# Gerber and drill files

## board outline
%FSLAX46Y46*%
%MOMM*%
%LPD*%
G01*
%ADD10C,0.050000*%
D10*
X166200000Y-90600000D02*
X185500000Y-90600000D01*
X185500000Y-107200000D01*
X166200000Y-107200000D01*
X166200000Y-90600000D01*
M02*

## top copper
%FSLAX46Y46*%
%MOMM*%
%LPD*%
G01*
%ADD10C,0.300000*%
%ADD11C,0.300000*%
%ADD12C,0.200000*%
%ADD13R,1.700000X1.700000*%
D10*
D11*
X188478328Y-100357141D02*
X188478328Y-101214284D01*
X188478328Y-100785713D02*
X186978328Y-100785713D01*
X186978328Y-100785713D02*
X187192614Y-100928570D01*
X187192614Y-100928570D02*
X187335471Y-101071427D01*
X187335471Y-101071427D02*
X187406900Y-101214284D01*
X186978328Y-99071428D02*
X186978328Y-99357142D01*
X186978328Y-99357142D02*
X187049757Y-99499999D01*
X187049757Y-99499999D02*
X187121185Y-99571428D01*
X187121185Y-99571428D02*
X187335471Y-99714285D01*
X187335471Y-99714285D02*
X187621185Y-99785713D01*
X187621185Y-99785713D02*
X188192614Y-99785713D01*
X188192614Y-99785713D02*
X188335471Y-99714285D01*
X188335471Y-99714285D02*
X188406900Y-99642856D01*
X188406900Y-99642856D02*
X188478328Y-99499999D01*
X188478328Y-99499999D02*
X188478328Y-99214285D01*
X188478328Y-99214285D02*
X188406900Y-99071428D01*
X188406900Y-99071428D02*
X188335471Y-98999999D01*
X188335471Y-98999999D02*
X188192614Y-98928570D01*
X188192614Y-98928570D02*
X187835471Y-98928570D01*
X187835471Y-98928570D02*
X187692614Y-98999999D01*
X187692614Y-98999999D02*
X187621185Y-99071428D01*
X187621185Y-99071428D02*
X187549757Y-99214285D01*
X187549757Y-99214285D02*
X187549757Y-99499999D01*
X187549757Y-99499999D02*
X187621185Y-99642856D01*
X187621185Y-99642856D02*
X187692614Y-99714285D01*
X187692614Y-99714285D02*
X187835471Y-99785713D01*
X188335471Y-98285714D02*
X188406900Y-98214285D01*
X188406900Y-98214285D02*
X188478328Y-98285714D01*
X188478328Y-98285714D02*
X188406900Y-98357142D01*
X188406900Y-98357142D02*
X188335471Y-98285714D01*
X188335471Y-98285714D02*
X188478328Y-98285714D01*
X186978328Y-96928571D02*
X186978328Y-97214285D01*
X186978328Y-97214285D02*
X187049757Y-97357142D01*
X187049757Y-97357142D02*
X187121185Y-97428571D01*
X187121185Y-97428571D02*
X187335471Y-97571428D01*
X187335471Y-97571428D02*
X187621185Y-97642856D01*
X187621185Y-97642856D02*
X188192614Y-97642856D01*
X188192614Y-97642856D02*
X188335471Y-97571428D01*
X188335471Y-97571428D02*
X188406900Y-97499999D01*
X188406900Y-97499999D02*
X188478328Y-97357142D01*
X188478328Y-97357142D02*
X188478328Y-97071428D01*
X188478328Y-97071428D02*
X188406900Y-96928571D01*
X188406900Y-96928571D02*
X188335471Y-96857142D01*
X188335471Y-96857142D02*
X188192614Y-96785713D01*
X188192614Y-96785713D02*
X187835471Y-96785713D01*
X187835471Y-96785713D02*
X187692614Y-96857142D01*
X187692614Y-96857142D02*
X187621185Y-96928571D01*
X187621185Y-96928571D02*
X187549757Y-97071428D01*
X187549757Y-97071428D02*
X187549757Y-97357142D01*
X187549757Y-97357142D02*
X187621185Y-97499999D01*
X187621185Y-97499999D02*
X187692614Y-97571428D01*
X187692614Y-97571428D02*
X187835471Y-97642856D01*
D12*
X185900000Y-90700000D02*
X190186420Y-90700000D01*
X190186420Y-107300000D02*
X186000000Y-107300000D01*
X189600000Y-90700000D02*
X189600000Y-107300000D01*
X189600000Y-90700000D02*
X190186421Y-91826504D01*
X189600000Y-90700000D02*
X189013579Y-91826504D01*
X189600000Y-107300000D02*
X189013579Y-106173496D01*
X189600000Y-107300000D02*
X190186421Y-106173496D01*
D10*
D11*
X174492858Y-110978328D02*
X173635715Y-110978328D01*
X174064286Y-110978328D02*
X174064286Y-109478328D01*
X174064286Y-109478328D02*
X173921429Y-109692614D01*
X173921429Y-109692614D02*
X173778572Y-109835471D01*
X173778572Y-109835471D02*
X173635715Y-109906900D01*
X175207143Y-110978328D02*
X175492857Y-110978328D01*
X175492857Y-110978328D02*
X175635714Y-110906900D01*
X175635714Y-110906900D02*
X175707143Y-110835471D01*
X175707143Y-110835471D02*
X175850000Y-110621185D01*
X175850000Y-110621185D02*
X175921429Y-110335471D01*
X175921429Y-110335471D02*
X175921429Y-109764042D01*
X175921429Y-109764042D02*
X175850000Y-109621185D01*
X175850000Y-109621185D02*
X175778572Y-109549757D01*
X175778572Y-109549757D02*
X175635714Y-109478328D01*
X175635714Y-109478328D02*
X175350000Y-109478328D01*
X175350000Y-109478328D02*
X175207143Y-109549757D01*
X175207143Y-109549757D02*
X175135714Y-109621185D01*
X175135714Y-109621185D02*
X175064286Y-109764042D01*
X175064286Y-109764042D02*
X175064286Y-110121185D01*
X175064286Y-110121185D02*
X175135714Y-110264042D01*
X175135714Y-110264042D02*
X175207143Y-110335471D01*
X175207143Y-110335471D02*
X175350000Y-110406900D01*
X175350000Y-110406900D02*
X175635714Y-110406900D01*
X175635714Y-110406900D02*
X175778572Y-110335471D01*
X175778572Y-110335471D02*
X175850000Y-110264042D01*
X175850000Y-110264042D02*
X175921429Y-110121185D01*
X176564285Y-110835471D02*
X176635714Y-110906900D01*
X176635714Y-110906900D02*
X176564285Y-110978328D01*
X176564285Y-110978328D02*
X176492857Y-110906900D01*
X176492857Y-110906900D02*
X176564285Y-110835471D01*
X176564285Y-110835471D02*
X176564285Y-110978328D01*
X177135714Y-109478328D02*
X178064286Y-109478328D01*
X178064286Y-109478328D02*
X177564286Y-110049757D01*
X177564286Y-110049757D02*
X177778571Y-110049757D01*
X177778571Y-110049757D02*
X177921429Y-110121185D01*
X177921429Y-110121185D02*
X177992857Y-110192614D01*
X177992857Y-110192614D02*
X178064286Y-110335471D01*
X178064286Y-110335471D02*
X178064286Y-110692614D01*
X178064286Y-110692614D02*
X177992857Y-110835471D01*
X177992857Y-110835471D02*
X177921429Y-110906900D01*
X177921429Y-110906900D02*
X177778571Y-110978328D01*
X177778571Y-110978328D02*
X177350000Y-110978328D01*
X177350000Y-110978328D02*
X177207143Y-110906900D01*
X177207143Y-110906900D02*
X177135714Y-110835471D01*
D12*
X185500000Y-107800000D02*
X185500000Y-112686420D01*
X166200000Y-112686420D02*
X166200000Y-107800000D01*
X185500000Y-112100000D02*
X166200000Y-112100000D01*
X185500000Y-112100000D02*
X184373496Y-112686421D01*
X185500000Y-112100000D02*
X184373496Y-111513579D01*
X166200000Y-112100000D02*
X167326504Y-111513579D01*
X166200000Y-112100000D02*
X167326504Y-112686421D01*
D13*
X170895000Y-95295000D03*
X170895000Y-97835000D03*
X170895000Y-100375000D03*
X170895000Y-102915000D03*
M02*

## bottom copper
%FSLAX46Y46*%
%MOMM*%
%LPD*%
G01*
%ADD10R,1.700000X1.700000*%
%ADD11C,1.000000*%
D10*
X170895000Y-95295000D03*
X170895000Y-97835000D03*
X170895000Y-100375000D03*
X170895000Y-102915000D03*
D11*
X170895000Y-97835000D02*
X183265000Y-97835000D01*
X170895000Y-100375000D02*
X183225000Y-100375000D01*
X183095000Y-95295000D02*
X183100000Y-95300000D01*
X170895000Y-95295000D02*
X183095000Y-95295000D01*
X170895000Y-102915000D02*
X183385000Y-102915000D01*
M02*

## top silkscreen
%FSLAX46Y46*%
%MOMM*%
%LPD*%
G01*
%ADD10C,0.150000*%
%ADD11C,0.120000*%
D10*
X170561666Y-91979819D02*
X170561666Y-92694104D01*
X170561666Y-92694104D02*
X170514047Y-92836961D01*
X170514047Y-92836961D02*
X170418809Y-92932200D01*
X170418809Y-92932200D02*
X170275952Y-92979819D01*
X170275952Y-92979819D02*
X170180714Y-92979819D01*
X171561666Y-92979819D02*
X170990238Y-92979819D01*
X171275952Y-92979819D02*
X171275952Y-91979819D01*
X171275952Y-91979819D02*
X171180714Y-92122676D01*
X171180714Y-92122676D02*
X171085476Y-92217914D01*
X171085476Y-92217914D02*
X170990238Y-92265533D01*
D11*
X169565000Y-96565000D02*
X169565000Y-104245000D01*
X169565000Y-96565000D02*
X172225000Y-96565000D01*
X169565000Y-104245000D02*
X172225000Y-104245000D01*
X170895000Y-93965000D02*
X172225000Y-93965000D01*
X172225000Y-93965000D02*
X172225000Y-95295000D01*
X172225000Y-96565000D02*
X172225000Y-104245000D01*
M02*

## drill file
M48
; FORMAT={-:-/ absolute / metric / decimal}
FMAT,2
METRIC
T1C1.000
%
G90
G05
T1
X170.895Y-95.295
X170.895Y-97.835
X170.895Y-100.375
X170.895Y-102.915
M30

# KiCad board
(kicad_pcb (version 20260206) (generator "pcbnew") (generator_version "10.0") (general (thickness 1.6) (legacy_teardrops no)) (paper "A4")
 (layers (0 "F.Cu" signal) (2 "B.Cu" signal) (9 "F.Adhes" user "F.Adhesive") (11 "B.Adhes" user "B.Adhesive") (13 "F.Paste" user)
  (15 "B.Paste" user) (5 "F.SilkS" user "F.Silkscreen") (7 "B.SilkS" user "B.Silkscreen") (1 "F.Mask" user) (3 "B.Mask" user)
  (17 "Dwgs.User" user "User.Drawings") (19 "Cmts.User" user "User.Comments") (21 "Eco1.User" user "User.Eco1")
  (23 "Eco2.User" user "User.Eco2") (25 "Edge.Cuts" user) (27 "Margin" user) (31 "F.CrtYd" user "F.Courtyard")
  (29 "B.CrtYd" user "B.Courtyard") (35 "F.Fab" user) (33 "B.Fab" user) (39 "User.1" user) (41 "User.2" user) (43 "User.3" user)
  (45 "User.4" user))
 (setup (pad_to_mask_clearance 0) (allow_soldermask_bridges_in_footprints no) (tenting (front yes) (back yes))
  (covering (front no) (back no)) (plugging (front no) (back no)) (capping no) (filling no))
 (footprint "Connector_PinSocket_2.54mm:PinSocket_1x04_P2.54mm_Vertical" (layer "F.Cu") (at 170.895 95.295)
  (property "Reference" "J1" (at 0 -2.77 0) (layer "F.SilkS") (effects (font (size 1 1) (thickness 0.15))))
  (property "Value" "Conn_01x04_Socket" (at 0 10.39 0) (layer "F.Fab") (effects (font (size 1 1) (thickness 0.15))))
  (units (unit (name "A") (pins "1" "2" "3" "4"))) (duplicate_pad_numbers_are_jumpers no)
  (fp_line (start -1.33 1.27) (end -1.33 8.95) (stroke (width 0.12) (type solid)) (layer "F.SilkS"))
  (fp_line (start -1.33 1.27) (end 1.33 1.27) (stroke (width 0.12) (type solid)) (layer "F.SilkS"))
  (fp_line (start -1.33 8.95) (end 1.33 8.95) (stroke (width 0.12) (type solid)) (layer "F.SilkS"))
  (fp_line (start 0 -1.33) (end 1.33 -1.33) (stroke (width 0.12) (type solid)) (layer "F.SilkS"))
  (fp_line (start 1.33 -1.33) (end 1.33 0) (stroke (width 0.12) (type solid)) (layer "F.SilkS"))
  (fp_line (start 1.33 1.27) (end 1.33 8.95) (stroke (width 0.12) (type solid)) (layer "F.SilkS"))
  (pad "1" thru_hole rect (at 0 0) (size 1.7 1.7) (drill 1) (layers "*.Cu" "*.Mask") (remove_unused_layers no)
   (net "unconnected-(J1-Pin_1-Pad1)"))
  (pad "2" thru_hole rect (at 0 2.54) (size 1.7 1.7) (drill 1) (layers "*.Cu" "*.Mask") (remove_unused_layers no)
   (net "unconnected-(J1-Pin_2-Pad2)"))
  (pad "3" thru_hole rect (at 0 5.08) (size 1.7 1.7) (drill 1) (layers "*.Cu" "*.Mask") (remove_unused_layers no)
   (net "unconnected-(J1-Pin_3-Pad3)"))
  (pad "4" thru_hole rect (at 0 7.62) (size 1.7 1.7) (drill 1) (layers "*.Cu" "*.Mask") (remove_unused_layers no)
   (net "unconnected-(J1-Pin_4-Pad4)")))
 (gr_rect (start 166.2 90.6) (end 185.5 107.2) (stroke (width 0.05) (type default)) (fill no) (layer "Edge.Cuts"))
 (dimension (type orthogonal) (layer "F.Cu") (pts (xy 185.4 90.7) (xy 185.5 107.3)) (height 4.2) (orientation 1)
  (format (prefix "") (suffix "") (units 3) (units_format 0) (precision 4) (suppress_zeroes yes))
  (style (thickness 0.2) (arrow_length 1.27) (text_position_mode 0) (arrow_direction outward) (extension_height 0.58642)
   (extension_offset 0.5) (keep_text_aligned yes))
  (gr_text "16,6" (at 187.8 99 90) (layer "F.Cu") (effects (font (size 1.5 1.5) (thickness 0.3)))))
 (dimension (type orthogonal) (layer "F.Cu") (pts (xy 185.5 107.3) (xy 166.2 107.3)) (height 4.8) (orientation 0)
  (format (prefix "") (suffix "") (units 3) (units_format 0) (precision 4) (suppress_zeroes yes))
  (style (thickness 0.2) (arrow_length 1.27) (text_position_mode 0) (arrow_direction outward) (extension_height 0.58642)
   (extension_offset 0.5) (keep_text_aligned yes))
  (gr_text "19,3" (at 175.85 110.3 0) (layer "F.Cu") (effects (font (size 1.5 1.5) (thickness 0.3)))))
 (segment (start 170.895 97.835) (end 183.265 97.835) (width 1) (layer "B.Cu") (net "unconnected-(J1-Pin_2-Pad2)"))
 (segment (start 170.895 100.375) (end 183.225 100.375) (width 1) (layer "B.Cu") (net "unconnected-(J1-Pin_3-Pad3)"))
 (segment (start 183.095 95.295) (end 183.1 95.3) (width 1) (layer "B.Cu") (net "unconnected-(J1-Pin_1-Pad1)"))
 (segment (start 170.895 95.295) (end 183.095 95.295) (width 1) (layer "B.Cu") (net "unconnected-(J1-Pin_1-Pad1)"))
 (segment (start 170.895 102.915) (end 183.385 102.915) (width 1) (layer "B.Cu") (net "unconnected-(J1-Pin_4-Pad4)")))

